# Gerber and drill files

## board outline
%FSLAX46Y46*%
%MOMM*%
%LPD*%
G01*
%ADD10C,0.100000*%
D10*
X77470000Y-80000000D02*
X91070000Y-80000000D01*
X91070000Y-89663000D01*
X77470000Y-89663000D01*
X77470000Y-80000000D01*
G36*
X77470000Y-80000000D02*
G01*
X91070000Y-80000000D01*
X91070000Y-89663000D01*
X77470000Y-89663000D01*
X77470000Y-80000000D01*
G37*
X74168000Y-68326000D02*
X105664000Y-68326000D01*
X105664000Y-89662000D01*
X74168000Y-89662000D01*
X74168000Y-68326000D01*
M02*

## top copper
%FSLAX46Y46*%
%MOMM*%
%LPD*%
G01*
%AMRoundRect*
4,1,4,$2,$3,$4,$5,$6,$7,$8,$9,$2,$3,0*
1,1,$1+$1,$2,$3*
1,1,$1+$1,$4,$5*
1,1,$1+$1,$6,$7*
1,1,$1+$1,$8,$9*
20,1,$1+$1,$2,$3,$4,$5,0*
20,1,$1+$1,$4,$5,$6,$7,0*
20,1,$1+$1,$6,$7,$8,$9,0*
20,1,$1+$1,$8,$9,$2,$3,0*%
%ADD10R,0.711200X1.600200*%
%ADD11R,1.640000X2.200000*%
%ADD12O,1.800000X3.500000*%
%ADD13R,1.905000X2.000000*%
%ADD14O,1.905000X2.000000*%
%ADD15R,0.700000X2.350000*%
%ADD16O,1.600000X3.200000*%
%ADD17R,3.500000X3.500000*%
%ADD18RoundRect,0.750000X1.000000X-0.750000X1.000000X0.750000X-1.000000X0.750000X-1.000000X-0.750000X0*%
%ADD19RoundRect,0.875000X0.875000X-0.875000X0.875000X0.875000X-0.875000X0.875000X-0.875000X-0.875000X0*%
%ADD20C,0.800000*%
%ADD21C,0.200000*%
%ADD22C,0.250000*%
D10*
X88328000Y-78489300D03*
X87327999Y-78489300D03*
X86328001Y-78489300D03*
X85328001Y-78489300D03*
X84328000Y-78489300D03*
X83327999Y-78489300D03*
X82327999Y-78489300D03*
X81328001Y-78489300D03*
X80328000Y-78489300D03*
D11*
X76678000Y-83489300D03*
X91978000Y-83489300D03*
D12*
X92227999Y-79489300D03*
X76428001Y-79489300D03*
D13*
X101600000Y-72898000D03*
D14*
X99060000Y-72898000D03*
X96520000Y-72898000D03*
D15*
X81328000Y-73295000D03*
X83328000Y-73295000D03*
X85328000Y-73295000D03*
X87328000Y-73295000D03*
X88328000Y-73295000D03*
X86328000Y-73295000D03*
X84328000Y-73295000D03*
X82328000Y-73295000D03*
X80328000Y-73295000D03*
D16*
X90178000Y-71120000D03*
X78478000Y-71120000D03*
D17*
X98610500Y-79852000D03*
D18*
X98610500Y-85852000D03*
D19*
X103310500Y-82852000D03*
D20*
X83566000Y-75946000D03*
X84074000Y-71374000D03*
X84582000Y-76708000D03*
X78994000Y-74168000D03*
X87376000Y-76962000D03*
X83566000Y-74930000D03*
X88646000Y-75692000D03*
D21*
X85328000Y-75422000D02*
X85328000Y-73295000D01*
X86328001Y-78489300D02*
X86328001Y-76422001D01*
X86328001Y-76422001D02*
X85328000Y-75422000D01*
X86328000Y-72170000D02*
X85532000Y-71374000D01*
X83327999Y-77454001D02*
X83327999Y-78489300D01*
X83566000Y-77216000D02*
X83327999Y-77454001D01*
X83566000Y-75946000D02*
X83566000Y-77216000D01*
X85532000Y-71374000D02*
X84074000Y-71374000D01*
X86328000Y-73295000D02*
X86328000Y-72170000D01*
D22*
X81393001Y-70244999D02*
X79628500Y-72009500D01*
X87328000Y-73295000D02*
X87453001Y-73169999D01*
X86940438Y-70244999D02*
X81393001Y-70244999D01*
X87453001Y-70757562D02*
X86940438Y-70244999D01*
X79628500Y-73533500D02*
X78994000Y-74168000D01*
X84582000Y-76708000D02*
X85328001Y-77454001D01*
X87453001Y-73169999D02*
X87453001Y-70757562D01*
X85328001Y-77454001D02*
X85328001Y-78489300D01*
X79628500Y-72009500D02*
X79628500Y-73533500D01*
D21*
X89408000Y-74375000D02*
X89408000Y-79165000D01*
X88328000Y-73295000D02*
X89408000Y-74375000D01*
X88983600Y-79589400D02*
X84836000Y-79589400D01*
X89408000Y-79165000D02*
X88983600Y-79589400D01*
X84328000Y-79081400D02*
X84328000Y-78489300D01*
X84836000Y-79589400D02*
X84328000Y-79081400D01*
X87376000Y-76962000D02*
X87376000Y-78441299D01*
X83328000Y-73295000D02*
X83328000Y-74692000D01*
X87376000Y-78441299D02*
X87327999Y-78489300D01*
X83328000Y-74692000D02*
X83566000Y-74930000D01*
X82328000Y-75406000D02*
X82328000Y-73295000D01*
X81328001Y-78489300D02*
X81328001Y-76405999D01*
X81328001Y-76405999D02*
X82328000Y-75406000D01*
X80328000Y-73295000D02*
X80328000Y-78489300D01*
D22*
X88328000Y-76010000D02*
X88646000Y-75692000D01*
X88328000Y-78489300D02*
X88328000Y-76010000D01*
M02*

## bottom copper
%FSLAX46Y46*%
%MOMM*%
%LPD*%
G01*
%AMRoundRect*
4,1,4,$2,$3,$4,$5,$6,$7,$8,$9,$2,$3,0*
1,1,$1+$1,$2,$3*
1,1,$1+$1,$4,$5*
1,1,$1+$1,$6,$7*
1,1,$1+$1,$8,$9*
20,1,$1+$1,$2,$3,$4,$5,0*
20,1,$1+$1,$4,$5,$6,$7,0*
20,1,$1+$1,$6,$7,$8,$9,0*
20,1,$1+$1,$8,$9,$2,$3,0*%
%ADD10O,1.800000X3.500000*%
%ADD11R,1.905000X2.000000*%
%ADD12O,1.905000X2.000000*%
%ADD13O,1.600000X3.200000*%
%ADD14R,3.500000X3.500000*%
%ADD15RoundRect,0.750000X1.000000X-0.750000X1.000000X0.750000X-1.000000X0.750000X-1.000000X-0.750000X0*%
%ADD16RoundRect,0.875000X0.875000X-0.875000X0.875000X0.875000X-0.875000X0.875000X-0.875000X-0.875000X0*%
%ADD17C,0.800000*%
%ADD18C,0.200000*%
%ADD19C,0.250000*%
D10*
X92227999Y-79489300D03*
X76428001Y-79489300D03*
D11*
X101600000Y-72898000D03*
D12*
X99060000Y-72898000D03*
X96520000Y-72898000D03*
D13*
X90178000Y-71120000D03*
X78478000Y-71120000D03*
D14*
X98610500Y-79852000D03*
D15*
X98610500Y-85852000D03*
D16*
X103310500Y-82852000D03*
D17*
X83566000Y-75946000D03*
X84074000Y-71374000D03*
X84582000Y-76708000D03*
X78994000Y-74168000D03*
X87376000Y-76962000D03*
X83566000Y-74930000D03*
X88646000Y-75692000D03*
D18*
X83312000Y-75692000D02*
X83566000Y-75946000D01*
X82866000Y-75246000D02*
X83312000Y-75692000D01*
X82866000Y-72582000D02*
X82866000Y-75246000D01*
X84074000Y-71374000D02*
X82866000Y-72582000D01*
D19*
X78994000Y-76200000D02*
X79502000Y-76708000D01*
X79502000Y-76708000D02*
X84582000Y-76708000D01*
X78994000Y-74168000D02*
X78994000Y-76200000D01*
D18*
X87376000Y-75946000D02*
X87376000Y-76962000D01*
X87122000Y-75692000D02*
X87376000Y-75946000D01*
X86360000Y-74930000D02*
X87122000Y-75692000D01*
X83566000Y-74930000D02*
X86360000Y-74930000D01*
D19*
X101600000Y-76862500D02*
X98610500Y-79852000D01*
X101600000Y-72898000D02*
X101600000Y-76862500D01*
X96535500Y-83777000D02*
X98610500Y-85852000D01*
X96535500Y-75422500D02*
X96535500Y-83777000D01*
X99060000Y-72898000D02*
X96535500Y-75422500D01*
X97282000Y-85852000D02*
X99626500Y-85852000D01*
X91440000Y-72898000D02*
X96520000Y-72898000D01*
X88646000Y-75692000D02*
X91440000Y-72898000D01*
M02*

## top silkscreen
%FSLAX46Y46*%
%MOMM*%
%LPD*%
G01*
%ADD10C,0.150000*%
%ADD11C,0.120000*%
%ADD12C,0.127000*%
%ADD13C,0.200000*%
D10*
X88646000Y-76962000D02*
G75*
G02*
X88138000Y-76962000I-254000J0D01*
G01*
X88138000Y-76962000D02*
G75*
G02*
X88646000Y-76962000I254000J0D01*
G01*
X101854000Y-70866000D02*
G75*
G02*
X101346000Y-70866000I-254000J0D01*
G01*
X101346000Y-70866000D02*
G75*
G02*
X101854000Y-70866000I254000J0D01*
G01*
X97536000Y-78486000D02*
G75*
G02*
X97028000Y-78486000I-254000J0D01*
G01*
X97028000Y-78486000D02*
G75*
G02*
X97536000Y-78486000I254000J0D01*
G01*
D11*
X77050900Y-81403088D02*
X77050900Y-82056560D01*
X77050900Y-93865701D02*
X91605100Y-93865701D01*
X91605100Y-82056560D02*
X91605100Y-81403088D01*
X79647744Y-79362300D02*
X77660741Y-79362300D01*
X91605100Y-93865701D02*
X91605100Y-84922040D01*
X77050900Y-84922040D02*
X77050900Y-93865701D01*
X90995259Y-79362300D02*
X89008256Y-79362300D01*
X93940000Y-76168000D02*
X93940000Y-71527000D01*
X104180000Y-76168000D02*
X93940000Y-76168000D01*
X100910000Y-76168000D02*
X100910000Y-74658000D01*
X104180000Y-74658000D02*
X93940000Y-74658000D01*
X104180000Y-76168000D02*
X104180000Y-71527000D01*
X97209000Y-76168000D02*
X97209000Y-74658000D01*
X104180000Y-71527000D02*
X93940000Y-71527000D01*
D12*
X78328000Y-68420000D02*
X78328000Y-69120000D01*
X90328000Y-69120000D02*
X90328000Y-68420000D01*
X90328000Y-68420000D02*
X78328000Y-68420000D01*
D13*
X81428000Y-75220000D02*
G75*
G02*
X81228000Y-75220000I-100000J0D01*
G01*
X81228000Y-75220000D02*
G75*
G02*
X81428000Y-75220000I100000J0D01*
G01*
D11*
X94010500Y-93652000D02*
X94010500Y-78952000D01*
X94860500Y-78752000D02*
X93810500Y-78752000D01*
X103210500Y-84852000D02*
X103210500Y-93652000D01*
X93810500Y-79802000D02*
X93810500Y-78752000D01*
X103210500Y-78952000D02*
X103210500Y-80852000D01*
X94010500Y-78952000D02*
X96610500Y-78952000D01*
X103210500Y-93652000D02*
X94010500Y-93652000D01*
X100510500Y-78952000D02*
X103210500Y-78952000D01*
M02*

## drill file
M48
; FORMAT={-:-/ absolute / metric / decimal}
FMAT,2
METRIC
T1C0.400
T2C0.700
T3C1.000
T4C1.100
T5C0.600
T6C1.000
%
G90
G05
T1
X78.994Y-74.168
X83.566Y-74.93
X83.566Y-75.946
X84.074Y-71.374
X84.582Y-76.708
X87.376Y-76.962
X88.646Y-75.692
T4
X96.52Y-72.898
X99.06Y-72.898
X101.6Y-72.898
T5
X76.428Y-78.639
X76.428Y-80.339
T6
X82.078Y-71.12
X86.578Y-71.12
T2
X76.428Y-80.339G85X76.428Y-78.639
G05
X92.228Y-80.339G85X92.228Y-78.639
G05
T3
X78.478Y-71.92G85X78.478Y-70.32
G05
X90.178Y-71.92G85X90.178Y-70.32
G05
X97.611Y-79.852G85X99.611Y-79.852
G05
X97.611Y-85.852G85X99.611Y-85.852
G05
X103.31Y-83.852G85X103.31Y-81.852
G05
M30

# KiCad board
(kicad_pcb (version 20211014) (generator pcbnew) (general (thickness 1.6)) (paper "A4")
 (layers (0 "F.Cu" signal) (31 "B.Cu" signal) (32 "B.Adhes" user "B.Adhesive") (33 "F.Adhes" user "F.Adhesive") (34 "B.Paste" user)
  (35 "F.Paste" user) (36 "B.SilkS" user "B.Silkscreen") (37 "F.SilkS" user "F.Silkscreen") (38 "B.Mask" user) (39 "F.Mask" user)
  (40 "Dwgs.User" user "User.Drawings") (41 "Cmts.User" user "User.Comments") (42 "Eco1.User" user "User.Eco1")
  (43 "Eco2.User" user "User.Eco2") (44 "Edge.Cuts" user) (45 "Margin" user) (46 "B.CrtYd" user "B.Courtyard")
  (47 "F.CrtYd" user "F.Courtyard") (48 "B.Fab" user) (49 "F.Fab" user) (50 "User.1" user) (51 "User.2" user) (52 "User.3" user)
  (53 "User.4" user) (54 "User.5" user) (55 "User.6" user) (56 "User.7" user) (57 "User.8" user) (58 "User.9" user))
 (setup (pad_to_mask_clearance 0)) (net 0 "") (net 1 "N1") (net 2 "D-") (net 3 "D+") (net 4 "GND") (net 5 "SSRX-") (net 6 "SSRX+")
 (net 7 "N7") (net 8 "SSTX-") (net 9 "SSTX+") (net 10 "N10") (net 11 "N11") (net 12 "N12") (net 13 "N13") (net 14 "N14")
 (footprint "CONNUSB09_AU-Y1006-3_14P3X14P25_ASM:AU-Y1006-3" (layer "F.Cu") (at 84.328 86.614)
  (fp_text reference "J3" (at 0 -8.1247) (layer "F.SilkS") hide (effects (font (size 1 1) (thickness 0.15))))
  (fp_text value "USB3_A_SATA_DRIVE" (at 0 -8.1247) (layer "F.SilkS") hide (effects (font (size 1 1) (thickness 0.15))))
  (fp_line (start -7.2771 -5.210912) (end -7.2771 -4.55744) (layer "F.SilkS") (width 0.12))
  (fp_line (start -7.2771 7.251701) (end 7.2771 7.251701) (layer "F.SilkS") (width 0.12))
  (fp_line (start 7.2771 -4.55744) (end 7.2771 -5.210912) (layer "F.SilkS") (width 0.12))
  (fp_line (start -4.680256 -7.2517) (end -6.667259 -7.2517) (layer "F.SilkS") (width 0.12))
  (fp_line (start 7.2771 7.251701) (end 7.2771 -1.69196) (layer "F.SilkS") (width 0.12))
  (fp_line (start -7.2771 -1.69196) (end -7.2771 7.251701) (layer "F.SilkS") (width 0.12))
  (fp_line (start 6.667259 -7.2517) (end 4.680256 -7.2517) (layer "F.SilkS") (width 0.12))
  (pad "" np_thru_hole circle (at -7.899999 -6.2747) (size 0.6 0.6) (drill 0.6) (layers *.Cu *.Mask))
  (pad "" np_thru_hole circle (at -7.899999 -7.9747) (size 0.6 0.6) (drill 0.6) (layers *.Cu *.Mask))
  (pad "1" smd rect (at 4 -8.1247) (size 0.7112 1.6002) (layers "F.Cu" "F.Paste" "F.Mask") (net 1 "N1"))
  (pad "2" smd rect (at 2.999999 -8.1247) (size 0.7112 1.6002) (layers "F.Cu" "F.Paste" "F.Mask") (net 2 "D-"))
  (pad "3" smd rect (at 2.000001 -8.1247) (size 0.7112 1.6002) (layers "F.Cu" "F.Paste" "F.Mask") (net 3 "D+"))
  (pad "4" smd rect (at 1.000001 -8.1247) (size 0.7112 1.6002) (layers "F.Cu" "F.Paste" "F.Mask") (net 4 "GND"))
  (pad "5" smd rect (at 0 -8.1247) (size 0.7112 1.6002) (layers "F.Cu" "F.Paste" "F.Mask") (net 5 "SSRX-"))
  (pad "6" smd rect (at -1.000001 -8.1247) (size 0.7112 1.6002) (layers "F.Cu" "F.Paste" "F.Mask") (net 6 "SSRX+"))
  (pad "7" smd rect (at -2.000001 -8.1247) (size 0.7112 1.6002) (layers "F.Cu" "F.Paste" "F.Mask") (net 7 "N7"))
  (pad "8" smd rect (at -2.999999 -8.1247) (size 0.7112 1.6002) (layers "F.Cu" "F.Paste" "F.Mask") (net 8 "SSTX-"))
  (pad "9" smd rect (at -4 -8.1247) (size 0.7112 1.6002) (layers "F.Cu" "F.Paste" "F.Mask") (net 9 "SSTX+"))
  (pad "10" smd rect (at -7.65 -3.1247) (size 1.64 2.2) (layers "F.Cu" "F.Paste" "F.Mask") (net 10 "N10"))
  (pad "11" smd rect (at 7.65 -3.1247) (size 1.64 2.2) (layers "F.Cu" "F.Paste" "F.Mask"))
  (pad "S_8" thru_hole oval (at 7.899999 -7.1247 90) (size 3.5 1.8) (drill oval 2.4 0.7) (layers *.Cu *.Mask))
  (pad "S_9" thru_hole oval (at -7.899999 -7.1247 90) (size 3.5 1.8) (drill oval 2.4 0.7) (layers *.Cu *.Mask)))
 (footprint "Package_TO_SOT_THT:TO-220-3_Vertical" (layer "F.Cu") (at 101.6 72.898 180)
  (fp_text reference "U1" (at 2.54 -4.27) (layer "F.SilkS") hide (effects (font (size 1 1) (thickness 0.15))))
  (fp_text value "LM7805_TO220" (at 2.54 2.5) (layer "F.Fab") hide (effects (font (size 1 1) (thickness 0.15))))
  (fp_line (start 7.66 -3.27) (end 7.66 1.371) (layer "F.SilkS") (width 0.12))
  (fp_line (start -2.58 -3.27) (end 7.66 -3.27) (layer "F.SilkS") (width 0.12))
  (fp_line (start 0.69 -3.27) (end 0.69 -1.76) (layer "F.SilkS") (width 0.12))
  (fp_line (start -2.58 -1.76) (end 7.66 -1.76) (layer "F.SilkS") (width 0.12))
  (fp_line (start -2.58 -3.27) (end -2.58 1.371) (layer "F.SilkS") (width 0.12))
  (fp_line (start 4.391 -3.27) (end 4.391 -1.76) (layer "F.SilkS") (width 0.12))
  (fp_line (start -2.58 1.371) (end 7.66 1.371) (layer "F.SilkS") (width 0.12))
  (pad "1" thru_hole rect (at 0 0 180) (size 1.905 2) (drill 1.1) (layers *.Cu *.Mask) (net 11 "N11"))
  (pad "2" thru_hole oval (at 2.54 0 180) (size 1.905 2) (drill 1.1) (layers *.Cu *.Mask) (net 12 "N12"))
  (pad "3" thru_hole oval (at 5.08 0 180) (size 1.905 2) (drill 1.1) (layers *.Cu *.Mask) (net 1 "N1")))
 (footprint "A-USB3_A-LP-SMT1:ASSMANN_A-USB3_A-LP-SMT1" (layer "F.Cu") (at 84.328 71.12 180)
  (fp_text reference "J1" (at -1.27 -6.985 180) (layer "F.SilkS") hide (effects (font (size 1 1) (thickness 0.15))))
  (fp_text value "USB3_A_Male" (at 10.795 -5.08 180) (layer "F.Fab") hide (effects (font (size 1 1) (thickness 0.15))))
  (fp_line (start 6 2.7) (end 6 2) (layer "F.SilkS") (width 0.127))
  (fp_line (start -6 2) (end -6 2.7) (layer "F.SilkS") (width 0.127))
  (fp_line (start -6 2.7) (end 6 2.7) (layer "F.SilkS") (width 0.127))
  (fp_circle (center 3 -4.1) (end 3.1 -4.1) (layer "F.SilkS") (width 0.2) (fill none))
  (pad "" np_thru_hole circle locked (at 2.25 0 180) (size 1 1) (drill 1) (layers *.Cu *.Mask))
  (pad "" np_thru_hole circle locked (at -2.25 0 180) (size 1 1) (drill 1) (layers *.Cu *.Mask))
  (pad "1" smd rect locked (at 3 -2.175 180) (size 0.7 2.35) (layers "F.Cu" "F.Paste" "F.Mask") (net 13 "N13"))
  (pad "2" smd rect locked (at 1 -2.175 180) (size 0.7 2.35) (layers "F.Cu" "F.Paste" "F.Mask") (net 2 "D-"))
  (pad "3" smd rect locked (at -1 -2.175 180) (size 0.7 2.35) (layers "F.Cu" "F.Paste" "F.Mask") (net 3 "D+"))
  (pad "4" smd rect locked (at -3 -2.175 180) (size 0.7 2.35) (layers "F.Cu" "F.Paste" "F.Mask") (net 4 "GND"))
  (pad "5" smd rect locked (at -4 -2.175 180) (size 0.7 2.35) (layers "F.Cu" "F.Paste" "F.Mask") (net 5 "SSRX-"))
  (pad "6" smd rect locked (at -2 -2.175 180) (size 0.7 2.35) (layers "F.Cu" "F.Paste" "F.Mask") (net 6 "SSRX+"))
  (pad "7" smd rect locked (at 0 -2.175 180) (size 0.7 2.35) (layers "F.Cu" "F.Paste" "F.Mask") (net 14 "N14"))
  (pad "8" smd rect locked (at 2 -2.175 180) (size 0.7 2.35) (layers "F.Cu" "F.Paste" "F.Mask") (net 8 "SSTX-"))
  (pad "9" smd rect locked (at 4 -2.175 180) (size 0.7 2.35) (layers "F.Cu" "F.Paste" "F.Mask") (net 9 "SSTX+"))
  (pad "S1" thru_hole oval locked (at -5.85 0 180) (size 1.6 3.2) (drill oval 1 2.6) (layers *.Cu *.Mask))
  (pad "S2" thru_hole oval locked (at 5.85 0 180) (size 1.6 3.2) (drill oval 1 2.6) (layers *.Cu *.Mask)))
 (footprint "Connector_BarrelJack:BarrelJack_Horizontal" (layer "F.Cu") (at 98.6105 79.852 90)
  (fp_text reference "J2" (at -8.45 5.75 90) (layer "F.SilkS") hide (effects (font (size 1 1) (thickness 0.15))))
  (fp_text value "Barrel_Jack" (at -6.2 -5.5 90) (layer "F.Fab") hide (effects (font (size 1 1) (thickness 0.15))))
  (fp_line (start -13.8 -4.6) (end 0.9 -4.6) (layer "F.SilkS") (width 0.12))
  (fp_line (start 1.1 -3.75) (end 1.1 -4.8) (layer "F.SilkS") (width 0.12))
  (fp_line (start -5 4.6) (end -13.8 4.6) (layer "F.SilkS") (width 0.12))
  (fp_line (start 0.05 -4.8) (end 1.1 -4.8) (layer "F.SilkS") (width 0.12))
  (fp_line (start 0.9 4.6) (end -1 4.6) (layer "F.SilkS") (width 0.12))
  (fp_line (start 0.9 -4.6) (end 0.9 -2) (layer "F.SilkS") (width 0.12))
  (fp_line (start -13.8 4.6) (end -13.8 -4.6) (layer "F.SilkS") (width 0.12))
  (fp_line (start 0.9 1.9) (end 0.9 4.6) (layer "F.SilkS") (width 0.12))
  (pad "1" thru_hole rect (at 0 0 90) (size 3.5 3.5) (drill oval 1 3) (layers *.Cu *.Mask) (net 11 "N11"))
  (pad "2" thru_hole roundrect (at -6 0 90) (size 3 3.5) (drill oval 1 3) (layers *.Cu *.Mask) (roundrect_rratio 0.25) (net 12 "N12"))
  (pad "3" thru_hole roundrect (at -3 4.7 90) (size 3.5 3.5) (drill oval 3 1) (layers *.Cu *.Mask) (roundrect_rratio 0.25)))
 (gr_circle (center 88.392 76.962) (end 88.392 76.708) (layer "F.SilkS") (width 0.15) (fill none))
 (gr_circle (center 101.6 70.866) (end 101.6 71.12) (layer "F.SilkS") (width 0.15) (fill none))
 (gr_circle (center 97.282 78.486) (end 97.282 78.232) (layer "F.SilkS") (width 0.15) (fill none))
 (gr_rect (start 77.47 80) (end 91.07 89.663) (layer "Edge.Cuts") (width 0.1) (fill solid))
 (gr_rect (start 105.664 89.662) (end 74.168 68.326) (layer "Edge.Cuts") (width 0.1) (fill none))
 (segment (start 85.328 75.422) (end 85.328 73.295) (width 0.2) (layer "F.Cu") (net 3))
 (segment (start 86.328001 78.4893) (end 86.328001 76.422001) (width 0.2) (layer "F.Cu") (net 3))
 (segment (start 86.328001 76.422001) (end 85.328 75.422) (width 0.2) (layer "F.Cu") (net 3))
 (segment (start 86.328 72.17) (end 85.532 71.374) (width 0.2) (layer "F.Cu") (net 6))
 (segment (start 83.327999 77.454001) (end 83.327999 78.4893) (width 0.2) (layer "F.Cu") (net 6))
 (segment (start 83.566 77.216) (end 83.327999 77.454001) (width 0.2) (layer "F.Cu") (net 6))
 (segment (start 83.566 75.946) (end 83.566 77.216) (width 0.2) (layer "F.Cu") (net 6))
 (segment (start 85.532 71.374) (end 84.074 71.374) (width 0.2) (layer "F.Cu") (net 6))
 (segment (start 86.328 73.295) (end 86.328 72.17) (width 0.2) (layer "F.Cu") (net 6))
 (via (at 83.566 75.946) (size 0.8) (drill 0.4) (layers "F.Cu" "B.Cu") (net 6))
 (via (at 84.074 71.374) (size 0.8) (drill 0.4) (layers "F.Cu" "B.Cu") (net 6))
 (segment (start 83.312 75.692) (end 83.566 75.946) (width 0.2) (layer "B.Cu") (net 6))
 (segment (start 82.866 75.246) (end 83.312 75.692) (width 0.2) (layer "B.Cu") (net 6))
 (segment (start 82.866 72.582) (end 82.866 75.246) (width 0.2) (layer "B.Cu") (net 6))
 (segment (start 84.074 71.374) (end 82.866 72.582) (width 0.2) (layer "B.Cu") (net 6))
 (segment (start 81.393001 70.244999) (end 79.6285 72.0095) (width 0.25) (layer "F.Cu") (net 4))
 (segment (start 87.328 73.295) (end 87.453001 73.169999) (width 0.25) (layer "F.Cu") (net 4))
 (segment (start 86.940438 70.244999) (end 81.393001 70.244999) (width 0.25) (layer "F.Cu") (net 4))
 (segment (start 87.453001 70.757562) (end 86.940438 70.244999) (width 0.25) (layer "F.Cu") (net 4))
 (segment (start 79.6285 73.5335) (end 78.994 74.168) (width 0.25) (layer "F.Cu") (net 4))
 (segment (start 84.582 76.708) (end 85.328001 77.454001) (width 0.25) (layer "F.Cu") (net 4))
 (segment (start 87.453001 73.169999) (end 87.453001 70.757562) (width 0.25) (layer "F.Cu") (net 4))
 (segment (start 85.328001 77.454001) (end 85.328001 78.4893) (width 0.25) (layer "F.Cu") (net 4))
 (segment (start 79.6285 72.0095) (end 79.6285 73.5335) (width 0.25) (layer "F.Cu") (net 4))
 (via (at 84.582 76.708) (size 0.8) (drill 0.4) (layers "F.Cu" "B.Cu") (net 4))
 (via (at 78.994 74.168) (size 0.8) (drill 0.4) (layers "F.Cu" "B.Cu") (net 4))
 (segment (start 78.994 76.2) (end 79.502 76.708) (width 0.25) (layer "B.Cu") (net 4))
 (segment (start 79.502 76.708) (end 84.582 76.708) (width 0.25) (layer "B.Cu") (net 4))
 (segment (start 78.994 74.168) (end 78.994 76.2) (width 0.25) (layer "B.Cu") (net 4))
 (segment (start 89.408 74.375) (end 89.408 79.165) (width 0.2) (layer "F.Cu") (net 5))
 (segment (start 88.328 73.295) (end 89.408 74.375) (width 0.2) (layer "F.Cu") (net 5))
 (segment (start 88.9836 79.5894) (end 84.836 79.5894) (width 0.2) (layer "F.Cu") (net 5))
 (segment (start 89.408 79.165) (end 88.9836 79.5894) (width 0.2) (layer "F.Cu") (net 5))
 (segment (start 84.328 79.0814) (end 84.328 78.4893) (width 0.2) (layer "F.Cu") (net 5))
 (segment (start 84.836 79.5894) (end 84.328 79.0814) (width 0.2) (layer "F.Cu") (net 5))
 (segment (start 87.376 76.962) (end 87.376 78.441299) (width 0.2) (layer "F.Cu") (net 2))
 (segment (start 83.328 73.295) (end 83.328 74.692) (width 0.2) (layer "F.Cu") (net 2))
 (segment (start 87.376 78.441299) (end 87.327999 78.4893) (width 0.2) (layer "F.Cu") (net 2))
 (segment (start 83.328 74.692) (end 83.566 74.93) (width 0.2) (layer "F.Cu") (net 2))
 (via (at 87.376 76.962) (size 0.8) (drill 0.4) (layers "F.Cu" "B.Cu") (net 2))
 (via (at 83.566 74.93) (size 0.8) (drill 0.4) (layers "F.Cu" "B.Cu") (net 2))
 (segment (start 87.376 75.946) (end 87.376 76.962) (width 0.2) (layer "B.Cu") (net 2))
 (segment (start 87.122 75.692) (end 87.376 75.946) (width 0.2) (layer "B.Cu") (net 2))
 (segment (start 86.36 74.93) (end 87.122 75.692) (width 0.2) (layer "B.Cu") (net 2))
 (segment (start 83.566 74.93) (end 86.36 74.93) (width 0.2) (layer "B.Cu") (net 2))
 (segment (start 82.328 75.406) (end 82.328 73.295) (width 0.2) (layer "F.Cu") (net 8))
 (segment (start 81.328001 78.4893) (end 81.328001 76.405999) (width 0.2) (layer "F.Cu") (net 8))
 (segment (start 81.328001 76.405999) (end 82.328 75.406) (width 0.2) (layer "F.Cu") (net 8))
 (segment (start 80.328 73.295) (end 80.328 78.4893) (width 0.2) (layer "F.Cu") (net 9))
 (segment (start 101.6 76.8625) (end 98.6105 79.852) (width 0.25) (layer "B.Cu") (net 11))
 (segment (start 101.6 72.898) (end 101.6 76.8625) (width 0.25) (layer "B.Cu") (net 11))
 (segment (start 96.5355 83.777) (end 98.6105 85.852) (width 0.25) (layer "B.Cu") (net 12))
 (segment (start 96.5355 75.4225) (end 96.5355 83.777) (width 0.25) (layer "B.Cu") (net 12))
 (segment (start 99.06 72.898) (end 96.5355 75.4225) (width 0.25) (layer "B.Cu") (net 12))
 (segment (start 97.282 85.852) (end 99.6265 85.852) (width 0.25) (layer "B.Cu") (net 12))
 (segment (start 88.328 76.01) (end 88.646 75.692) (width 0.25) (layer "F.Cu") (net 1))
 (segment (start 88.328 78.4893) (end 88.328 76.01) (width 0.25) (layer "F.Cu") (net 1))
 (via (at 88.646 75.692) (size 0.8) (drill 0.4) (layers "F.Cu" "B.Cu") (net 1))
 (segment (start 91.44 72.898) (end 96.52 72.898) (width 0.25) (layer "B.Cu") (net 1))
 (segment (start 88.646 75.692) (end 91.44 72.898) (width 0.25) (layer "B.Cu") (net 1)))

